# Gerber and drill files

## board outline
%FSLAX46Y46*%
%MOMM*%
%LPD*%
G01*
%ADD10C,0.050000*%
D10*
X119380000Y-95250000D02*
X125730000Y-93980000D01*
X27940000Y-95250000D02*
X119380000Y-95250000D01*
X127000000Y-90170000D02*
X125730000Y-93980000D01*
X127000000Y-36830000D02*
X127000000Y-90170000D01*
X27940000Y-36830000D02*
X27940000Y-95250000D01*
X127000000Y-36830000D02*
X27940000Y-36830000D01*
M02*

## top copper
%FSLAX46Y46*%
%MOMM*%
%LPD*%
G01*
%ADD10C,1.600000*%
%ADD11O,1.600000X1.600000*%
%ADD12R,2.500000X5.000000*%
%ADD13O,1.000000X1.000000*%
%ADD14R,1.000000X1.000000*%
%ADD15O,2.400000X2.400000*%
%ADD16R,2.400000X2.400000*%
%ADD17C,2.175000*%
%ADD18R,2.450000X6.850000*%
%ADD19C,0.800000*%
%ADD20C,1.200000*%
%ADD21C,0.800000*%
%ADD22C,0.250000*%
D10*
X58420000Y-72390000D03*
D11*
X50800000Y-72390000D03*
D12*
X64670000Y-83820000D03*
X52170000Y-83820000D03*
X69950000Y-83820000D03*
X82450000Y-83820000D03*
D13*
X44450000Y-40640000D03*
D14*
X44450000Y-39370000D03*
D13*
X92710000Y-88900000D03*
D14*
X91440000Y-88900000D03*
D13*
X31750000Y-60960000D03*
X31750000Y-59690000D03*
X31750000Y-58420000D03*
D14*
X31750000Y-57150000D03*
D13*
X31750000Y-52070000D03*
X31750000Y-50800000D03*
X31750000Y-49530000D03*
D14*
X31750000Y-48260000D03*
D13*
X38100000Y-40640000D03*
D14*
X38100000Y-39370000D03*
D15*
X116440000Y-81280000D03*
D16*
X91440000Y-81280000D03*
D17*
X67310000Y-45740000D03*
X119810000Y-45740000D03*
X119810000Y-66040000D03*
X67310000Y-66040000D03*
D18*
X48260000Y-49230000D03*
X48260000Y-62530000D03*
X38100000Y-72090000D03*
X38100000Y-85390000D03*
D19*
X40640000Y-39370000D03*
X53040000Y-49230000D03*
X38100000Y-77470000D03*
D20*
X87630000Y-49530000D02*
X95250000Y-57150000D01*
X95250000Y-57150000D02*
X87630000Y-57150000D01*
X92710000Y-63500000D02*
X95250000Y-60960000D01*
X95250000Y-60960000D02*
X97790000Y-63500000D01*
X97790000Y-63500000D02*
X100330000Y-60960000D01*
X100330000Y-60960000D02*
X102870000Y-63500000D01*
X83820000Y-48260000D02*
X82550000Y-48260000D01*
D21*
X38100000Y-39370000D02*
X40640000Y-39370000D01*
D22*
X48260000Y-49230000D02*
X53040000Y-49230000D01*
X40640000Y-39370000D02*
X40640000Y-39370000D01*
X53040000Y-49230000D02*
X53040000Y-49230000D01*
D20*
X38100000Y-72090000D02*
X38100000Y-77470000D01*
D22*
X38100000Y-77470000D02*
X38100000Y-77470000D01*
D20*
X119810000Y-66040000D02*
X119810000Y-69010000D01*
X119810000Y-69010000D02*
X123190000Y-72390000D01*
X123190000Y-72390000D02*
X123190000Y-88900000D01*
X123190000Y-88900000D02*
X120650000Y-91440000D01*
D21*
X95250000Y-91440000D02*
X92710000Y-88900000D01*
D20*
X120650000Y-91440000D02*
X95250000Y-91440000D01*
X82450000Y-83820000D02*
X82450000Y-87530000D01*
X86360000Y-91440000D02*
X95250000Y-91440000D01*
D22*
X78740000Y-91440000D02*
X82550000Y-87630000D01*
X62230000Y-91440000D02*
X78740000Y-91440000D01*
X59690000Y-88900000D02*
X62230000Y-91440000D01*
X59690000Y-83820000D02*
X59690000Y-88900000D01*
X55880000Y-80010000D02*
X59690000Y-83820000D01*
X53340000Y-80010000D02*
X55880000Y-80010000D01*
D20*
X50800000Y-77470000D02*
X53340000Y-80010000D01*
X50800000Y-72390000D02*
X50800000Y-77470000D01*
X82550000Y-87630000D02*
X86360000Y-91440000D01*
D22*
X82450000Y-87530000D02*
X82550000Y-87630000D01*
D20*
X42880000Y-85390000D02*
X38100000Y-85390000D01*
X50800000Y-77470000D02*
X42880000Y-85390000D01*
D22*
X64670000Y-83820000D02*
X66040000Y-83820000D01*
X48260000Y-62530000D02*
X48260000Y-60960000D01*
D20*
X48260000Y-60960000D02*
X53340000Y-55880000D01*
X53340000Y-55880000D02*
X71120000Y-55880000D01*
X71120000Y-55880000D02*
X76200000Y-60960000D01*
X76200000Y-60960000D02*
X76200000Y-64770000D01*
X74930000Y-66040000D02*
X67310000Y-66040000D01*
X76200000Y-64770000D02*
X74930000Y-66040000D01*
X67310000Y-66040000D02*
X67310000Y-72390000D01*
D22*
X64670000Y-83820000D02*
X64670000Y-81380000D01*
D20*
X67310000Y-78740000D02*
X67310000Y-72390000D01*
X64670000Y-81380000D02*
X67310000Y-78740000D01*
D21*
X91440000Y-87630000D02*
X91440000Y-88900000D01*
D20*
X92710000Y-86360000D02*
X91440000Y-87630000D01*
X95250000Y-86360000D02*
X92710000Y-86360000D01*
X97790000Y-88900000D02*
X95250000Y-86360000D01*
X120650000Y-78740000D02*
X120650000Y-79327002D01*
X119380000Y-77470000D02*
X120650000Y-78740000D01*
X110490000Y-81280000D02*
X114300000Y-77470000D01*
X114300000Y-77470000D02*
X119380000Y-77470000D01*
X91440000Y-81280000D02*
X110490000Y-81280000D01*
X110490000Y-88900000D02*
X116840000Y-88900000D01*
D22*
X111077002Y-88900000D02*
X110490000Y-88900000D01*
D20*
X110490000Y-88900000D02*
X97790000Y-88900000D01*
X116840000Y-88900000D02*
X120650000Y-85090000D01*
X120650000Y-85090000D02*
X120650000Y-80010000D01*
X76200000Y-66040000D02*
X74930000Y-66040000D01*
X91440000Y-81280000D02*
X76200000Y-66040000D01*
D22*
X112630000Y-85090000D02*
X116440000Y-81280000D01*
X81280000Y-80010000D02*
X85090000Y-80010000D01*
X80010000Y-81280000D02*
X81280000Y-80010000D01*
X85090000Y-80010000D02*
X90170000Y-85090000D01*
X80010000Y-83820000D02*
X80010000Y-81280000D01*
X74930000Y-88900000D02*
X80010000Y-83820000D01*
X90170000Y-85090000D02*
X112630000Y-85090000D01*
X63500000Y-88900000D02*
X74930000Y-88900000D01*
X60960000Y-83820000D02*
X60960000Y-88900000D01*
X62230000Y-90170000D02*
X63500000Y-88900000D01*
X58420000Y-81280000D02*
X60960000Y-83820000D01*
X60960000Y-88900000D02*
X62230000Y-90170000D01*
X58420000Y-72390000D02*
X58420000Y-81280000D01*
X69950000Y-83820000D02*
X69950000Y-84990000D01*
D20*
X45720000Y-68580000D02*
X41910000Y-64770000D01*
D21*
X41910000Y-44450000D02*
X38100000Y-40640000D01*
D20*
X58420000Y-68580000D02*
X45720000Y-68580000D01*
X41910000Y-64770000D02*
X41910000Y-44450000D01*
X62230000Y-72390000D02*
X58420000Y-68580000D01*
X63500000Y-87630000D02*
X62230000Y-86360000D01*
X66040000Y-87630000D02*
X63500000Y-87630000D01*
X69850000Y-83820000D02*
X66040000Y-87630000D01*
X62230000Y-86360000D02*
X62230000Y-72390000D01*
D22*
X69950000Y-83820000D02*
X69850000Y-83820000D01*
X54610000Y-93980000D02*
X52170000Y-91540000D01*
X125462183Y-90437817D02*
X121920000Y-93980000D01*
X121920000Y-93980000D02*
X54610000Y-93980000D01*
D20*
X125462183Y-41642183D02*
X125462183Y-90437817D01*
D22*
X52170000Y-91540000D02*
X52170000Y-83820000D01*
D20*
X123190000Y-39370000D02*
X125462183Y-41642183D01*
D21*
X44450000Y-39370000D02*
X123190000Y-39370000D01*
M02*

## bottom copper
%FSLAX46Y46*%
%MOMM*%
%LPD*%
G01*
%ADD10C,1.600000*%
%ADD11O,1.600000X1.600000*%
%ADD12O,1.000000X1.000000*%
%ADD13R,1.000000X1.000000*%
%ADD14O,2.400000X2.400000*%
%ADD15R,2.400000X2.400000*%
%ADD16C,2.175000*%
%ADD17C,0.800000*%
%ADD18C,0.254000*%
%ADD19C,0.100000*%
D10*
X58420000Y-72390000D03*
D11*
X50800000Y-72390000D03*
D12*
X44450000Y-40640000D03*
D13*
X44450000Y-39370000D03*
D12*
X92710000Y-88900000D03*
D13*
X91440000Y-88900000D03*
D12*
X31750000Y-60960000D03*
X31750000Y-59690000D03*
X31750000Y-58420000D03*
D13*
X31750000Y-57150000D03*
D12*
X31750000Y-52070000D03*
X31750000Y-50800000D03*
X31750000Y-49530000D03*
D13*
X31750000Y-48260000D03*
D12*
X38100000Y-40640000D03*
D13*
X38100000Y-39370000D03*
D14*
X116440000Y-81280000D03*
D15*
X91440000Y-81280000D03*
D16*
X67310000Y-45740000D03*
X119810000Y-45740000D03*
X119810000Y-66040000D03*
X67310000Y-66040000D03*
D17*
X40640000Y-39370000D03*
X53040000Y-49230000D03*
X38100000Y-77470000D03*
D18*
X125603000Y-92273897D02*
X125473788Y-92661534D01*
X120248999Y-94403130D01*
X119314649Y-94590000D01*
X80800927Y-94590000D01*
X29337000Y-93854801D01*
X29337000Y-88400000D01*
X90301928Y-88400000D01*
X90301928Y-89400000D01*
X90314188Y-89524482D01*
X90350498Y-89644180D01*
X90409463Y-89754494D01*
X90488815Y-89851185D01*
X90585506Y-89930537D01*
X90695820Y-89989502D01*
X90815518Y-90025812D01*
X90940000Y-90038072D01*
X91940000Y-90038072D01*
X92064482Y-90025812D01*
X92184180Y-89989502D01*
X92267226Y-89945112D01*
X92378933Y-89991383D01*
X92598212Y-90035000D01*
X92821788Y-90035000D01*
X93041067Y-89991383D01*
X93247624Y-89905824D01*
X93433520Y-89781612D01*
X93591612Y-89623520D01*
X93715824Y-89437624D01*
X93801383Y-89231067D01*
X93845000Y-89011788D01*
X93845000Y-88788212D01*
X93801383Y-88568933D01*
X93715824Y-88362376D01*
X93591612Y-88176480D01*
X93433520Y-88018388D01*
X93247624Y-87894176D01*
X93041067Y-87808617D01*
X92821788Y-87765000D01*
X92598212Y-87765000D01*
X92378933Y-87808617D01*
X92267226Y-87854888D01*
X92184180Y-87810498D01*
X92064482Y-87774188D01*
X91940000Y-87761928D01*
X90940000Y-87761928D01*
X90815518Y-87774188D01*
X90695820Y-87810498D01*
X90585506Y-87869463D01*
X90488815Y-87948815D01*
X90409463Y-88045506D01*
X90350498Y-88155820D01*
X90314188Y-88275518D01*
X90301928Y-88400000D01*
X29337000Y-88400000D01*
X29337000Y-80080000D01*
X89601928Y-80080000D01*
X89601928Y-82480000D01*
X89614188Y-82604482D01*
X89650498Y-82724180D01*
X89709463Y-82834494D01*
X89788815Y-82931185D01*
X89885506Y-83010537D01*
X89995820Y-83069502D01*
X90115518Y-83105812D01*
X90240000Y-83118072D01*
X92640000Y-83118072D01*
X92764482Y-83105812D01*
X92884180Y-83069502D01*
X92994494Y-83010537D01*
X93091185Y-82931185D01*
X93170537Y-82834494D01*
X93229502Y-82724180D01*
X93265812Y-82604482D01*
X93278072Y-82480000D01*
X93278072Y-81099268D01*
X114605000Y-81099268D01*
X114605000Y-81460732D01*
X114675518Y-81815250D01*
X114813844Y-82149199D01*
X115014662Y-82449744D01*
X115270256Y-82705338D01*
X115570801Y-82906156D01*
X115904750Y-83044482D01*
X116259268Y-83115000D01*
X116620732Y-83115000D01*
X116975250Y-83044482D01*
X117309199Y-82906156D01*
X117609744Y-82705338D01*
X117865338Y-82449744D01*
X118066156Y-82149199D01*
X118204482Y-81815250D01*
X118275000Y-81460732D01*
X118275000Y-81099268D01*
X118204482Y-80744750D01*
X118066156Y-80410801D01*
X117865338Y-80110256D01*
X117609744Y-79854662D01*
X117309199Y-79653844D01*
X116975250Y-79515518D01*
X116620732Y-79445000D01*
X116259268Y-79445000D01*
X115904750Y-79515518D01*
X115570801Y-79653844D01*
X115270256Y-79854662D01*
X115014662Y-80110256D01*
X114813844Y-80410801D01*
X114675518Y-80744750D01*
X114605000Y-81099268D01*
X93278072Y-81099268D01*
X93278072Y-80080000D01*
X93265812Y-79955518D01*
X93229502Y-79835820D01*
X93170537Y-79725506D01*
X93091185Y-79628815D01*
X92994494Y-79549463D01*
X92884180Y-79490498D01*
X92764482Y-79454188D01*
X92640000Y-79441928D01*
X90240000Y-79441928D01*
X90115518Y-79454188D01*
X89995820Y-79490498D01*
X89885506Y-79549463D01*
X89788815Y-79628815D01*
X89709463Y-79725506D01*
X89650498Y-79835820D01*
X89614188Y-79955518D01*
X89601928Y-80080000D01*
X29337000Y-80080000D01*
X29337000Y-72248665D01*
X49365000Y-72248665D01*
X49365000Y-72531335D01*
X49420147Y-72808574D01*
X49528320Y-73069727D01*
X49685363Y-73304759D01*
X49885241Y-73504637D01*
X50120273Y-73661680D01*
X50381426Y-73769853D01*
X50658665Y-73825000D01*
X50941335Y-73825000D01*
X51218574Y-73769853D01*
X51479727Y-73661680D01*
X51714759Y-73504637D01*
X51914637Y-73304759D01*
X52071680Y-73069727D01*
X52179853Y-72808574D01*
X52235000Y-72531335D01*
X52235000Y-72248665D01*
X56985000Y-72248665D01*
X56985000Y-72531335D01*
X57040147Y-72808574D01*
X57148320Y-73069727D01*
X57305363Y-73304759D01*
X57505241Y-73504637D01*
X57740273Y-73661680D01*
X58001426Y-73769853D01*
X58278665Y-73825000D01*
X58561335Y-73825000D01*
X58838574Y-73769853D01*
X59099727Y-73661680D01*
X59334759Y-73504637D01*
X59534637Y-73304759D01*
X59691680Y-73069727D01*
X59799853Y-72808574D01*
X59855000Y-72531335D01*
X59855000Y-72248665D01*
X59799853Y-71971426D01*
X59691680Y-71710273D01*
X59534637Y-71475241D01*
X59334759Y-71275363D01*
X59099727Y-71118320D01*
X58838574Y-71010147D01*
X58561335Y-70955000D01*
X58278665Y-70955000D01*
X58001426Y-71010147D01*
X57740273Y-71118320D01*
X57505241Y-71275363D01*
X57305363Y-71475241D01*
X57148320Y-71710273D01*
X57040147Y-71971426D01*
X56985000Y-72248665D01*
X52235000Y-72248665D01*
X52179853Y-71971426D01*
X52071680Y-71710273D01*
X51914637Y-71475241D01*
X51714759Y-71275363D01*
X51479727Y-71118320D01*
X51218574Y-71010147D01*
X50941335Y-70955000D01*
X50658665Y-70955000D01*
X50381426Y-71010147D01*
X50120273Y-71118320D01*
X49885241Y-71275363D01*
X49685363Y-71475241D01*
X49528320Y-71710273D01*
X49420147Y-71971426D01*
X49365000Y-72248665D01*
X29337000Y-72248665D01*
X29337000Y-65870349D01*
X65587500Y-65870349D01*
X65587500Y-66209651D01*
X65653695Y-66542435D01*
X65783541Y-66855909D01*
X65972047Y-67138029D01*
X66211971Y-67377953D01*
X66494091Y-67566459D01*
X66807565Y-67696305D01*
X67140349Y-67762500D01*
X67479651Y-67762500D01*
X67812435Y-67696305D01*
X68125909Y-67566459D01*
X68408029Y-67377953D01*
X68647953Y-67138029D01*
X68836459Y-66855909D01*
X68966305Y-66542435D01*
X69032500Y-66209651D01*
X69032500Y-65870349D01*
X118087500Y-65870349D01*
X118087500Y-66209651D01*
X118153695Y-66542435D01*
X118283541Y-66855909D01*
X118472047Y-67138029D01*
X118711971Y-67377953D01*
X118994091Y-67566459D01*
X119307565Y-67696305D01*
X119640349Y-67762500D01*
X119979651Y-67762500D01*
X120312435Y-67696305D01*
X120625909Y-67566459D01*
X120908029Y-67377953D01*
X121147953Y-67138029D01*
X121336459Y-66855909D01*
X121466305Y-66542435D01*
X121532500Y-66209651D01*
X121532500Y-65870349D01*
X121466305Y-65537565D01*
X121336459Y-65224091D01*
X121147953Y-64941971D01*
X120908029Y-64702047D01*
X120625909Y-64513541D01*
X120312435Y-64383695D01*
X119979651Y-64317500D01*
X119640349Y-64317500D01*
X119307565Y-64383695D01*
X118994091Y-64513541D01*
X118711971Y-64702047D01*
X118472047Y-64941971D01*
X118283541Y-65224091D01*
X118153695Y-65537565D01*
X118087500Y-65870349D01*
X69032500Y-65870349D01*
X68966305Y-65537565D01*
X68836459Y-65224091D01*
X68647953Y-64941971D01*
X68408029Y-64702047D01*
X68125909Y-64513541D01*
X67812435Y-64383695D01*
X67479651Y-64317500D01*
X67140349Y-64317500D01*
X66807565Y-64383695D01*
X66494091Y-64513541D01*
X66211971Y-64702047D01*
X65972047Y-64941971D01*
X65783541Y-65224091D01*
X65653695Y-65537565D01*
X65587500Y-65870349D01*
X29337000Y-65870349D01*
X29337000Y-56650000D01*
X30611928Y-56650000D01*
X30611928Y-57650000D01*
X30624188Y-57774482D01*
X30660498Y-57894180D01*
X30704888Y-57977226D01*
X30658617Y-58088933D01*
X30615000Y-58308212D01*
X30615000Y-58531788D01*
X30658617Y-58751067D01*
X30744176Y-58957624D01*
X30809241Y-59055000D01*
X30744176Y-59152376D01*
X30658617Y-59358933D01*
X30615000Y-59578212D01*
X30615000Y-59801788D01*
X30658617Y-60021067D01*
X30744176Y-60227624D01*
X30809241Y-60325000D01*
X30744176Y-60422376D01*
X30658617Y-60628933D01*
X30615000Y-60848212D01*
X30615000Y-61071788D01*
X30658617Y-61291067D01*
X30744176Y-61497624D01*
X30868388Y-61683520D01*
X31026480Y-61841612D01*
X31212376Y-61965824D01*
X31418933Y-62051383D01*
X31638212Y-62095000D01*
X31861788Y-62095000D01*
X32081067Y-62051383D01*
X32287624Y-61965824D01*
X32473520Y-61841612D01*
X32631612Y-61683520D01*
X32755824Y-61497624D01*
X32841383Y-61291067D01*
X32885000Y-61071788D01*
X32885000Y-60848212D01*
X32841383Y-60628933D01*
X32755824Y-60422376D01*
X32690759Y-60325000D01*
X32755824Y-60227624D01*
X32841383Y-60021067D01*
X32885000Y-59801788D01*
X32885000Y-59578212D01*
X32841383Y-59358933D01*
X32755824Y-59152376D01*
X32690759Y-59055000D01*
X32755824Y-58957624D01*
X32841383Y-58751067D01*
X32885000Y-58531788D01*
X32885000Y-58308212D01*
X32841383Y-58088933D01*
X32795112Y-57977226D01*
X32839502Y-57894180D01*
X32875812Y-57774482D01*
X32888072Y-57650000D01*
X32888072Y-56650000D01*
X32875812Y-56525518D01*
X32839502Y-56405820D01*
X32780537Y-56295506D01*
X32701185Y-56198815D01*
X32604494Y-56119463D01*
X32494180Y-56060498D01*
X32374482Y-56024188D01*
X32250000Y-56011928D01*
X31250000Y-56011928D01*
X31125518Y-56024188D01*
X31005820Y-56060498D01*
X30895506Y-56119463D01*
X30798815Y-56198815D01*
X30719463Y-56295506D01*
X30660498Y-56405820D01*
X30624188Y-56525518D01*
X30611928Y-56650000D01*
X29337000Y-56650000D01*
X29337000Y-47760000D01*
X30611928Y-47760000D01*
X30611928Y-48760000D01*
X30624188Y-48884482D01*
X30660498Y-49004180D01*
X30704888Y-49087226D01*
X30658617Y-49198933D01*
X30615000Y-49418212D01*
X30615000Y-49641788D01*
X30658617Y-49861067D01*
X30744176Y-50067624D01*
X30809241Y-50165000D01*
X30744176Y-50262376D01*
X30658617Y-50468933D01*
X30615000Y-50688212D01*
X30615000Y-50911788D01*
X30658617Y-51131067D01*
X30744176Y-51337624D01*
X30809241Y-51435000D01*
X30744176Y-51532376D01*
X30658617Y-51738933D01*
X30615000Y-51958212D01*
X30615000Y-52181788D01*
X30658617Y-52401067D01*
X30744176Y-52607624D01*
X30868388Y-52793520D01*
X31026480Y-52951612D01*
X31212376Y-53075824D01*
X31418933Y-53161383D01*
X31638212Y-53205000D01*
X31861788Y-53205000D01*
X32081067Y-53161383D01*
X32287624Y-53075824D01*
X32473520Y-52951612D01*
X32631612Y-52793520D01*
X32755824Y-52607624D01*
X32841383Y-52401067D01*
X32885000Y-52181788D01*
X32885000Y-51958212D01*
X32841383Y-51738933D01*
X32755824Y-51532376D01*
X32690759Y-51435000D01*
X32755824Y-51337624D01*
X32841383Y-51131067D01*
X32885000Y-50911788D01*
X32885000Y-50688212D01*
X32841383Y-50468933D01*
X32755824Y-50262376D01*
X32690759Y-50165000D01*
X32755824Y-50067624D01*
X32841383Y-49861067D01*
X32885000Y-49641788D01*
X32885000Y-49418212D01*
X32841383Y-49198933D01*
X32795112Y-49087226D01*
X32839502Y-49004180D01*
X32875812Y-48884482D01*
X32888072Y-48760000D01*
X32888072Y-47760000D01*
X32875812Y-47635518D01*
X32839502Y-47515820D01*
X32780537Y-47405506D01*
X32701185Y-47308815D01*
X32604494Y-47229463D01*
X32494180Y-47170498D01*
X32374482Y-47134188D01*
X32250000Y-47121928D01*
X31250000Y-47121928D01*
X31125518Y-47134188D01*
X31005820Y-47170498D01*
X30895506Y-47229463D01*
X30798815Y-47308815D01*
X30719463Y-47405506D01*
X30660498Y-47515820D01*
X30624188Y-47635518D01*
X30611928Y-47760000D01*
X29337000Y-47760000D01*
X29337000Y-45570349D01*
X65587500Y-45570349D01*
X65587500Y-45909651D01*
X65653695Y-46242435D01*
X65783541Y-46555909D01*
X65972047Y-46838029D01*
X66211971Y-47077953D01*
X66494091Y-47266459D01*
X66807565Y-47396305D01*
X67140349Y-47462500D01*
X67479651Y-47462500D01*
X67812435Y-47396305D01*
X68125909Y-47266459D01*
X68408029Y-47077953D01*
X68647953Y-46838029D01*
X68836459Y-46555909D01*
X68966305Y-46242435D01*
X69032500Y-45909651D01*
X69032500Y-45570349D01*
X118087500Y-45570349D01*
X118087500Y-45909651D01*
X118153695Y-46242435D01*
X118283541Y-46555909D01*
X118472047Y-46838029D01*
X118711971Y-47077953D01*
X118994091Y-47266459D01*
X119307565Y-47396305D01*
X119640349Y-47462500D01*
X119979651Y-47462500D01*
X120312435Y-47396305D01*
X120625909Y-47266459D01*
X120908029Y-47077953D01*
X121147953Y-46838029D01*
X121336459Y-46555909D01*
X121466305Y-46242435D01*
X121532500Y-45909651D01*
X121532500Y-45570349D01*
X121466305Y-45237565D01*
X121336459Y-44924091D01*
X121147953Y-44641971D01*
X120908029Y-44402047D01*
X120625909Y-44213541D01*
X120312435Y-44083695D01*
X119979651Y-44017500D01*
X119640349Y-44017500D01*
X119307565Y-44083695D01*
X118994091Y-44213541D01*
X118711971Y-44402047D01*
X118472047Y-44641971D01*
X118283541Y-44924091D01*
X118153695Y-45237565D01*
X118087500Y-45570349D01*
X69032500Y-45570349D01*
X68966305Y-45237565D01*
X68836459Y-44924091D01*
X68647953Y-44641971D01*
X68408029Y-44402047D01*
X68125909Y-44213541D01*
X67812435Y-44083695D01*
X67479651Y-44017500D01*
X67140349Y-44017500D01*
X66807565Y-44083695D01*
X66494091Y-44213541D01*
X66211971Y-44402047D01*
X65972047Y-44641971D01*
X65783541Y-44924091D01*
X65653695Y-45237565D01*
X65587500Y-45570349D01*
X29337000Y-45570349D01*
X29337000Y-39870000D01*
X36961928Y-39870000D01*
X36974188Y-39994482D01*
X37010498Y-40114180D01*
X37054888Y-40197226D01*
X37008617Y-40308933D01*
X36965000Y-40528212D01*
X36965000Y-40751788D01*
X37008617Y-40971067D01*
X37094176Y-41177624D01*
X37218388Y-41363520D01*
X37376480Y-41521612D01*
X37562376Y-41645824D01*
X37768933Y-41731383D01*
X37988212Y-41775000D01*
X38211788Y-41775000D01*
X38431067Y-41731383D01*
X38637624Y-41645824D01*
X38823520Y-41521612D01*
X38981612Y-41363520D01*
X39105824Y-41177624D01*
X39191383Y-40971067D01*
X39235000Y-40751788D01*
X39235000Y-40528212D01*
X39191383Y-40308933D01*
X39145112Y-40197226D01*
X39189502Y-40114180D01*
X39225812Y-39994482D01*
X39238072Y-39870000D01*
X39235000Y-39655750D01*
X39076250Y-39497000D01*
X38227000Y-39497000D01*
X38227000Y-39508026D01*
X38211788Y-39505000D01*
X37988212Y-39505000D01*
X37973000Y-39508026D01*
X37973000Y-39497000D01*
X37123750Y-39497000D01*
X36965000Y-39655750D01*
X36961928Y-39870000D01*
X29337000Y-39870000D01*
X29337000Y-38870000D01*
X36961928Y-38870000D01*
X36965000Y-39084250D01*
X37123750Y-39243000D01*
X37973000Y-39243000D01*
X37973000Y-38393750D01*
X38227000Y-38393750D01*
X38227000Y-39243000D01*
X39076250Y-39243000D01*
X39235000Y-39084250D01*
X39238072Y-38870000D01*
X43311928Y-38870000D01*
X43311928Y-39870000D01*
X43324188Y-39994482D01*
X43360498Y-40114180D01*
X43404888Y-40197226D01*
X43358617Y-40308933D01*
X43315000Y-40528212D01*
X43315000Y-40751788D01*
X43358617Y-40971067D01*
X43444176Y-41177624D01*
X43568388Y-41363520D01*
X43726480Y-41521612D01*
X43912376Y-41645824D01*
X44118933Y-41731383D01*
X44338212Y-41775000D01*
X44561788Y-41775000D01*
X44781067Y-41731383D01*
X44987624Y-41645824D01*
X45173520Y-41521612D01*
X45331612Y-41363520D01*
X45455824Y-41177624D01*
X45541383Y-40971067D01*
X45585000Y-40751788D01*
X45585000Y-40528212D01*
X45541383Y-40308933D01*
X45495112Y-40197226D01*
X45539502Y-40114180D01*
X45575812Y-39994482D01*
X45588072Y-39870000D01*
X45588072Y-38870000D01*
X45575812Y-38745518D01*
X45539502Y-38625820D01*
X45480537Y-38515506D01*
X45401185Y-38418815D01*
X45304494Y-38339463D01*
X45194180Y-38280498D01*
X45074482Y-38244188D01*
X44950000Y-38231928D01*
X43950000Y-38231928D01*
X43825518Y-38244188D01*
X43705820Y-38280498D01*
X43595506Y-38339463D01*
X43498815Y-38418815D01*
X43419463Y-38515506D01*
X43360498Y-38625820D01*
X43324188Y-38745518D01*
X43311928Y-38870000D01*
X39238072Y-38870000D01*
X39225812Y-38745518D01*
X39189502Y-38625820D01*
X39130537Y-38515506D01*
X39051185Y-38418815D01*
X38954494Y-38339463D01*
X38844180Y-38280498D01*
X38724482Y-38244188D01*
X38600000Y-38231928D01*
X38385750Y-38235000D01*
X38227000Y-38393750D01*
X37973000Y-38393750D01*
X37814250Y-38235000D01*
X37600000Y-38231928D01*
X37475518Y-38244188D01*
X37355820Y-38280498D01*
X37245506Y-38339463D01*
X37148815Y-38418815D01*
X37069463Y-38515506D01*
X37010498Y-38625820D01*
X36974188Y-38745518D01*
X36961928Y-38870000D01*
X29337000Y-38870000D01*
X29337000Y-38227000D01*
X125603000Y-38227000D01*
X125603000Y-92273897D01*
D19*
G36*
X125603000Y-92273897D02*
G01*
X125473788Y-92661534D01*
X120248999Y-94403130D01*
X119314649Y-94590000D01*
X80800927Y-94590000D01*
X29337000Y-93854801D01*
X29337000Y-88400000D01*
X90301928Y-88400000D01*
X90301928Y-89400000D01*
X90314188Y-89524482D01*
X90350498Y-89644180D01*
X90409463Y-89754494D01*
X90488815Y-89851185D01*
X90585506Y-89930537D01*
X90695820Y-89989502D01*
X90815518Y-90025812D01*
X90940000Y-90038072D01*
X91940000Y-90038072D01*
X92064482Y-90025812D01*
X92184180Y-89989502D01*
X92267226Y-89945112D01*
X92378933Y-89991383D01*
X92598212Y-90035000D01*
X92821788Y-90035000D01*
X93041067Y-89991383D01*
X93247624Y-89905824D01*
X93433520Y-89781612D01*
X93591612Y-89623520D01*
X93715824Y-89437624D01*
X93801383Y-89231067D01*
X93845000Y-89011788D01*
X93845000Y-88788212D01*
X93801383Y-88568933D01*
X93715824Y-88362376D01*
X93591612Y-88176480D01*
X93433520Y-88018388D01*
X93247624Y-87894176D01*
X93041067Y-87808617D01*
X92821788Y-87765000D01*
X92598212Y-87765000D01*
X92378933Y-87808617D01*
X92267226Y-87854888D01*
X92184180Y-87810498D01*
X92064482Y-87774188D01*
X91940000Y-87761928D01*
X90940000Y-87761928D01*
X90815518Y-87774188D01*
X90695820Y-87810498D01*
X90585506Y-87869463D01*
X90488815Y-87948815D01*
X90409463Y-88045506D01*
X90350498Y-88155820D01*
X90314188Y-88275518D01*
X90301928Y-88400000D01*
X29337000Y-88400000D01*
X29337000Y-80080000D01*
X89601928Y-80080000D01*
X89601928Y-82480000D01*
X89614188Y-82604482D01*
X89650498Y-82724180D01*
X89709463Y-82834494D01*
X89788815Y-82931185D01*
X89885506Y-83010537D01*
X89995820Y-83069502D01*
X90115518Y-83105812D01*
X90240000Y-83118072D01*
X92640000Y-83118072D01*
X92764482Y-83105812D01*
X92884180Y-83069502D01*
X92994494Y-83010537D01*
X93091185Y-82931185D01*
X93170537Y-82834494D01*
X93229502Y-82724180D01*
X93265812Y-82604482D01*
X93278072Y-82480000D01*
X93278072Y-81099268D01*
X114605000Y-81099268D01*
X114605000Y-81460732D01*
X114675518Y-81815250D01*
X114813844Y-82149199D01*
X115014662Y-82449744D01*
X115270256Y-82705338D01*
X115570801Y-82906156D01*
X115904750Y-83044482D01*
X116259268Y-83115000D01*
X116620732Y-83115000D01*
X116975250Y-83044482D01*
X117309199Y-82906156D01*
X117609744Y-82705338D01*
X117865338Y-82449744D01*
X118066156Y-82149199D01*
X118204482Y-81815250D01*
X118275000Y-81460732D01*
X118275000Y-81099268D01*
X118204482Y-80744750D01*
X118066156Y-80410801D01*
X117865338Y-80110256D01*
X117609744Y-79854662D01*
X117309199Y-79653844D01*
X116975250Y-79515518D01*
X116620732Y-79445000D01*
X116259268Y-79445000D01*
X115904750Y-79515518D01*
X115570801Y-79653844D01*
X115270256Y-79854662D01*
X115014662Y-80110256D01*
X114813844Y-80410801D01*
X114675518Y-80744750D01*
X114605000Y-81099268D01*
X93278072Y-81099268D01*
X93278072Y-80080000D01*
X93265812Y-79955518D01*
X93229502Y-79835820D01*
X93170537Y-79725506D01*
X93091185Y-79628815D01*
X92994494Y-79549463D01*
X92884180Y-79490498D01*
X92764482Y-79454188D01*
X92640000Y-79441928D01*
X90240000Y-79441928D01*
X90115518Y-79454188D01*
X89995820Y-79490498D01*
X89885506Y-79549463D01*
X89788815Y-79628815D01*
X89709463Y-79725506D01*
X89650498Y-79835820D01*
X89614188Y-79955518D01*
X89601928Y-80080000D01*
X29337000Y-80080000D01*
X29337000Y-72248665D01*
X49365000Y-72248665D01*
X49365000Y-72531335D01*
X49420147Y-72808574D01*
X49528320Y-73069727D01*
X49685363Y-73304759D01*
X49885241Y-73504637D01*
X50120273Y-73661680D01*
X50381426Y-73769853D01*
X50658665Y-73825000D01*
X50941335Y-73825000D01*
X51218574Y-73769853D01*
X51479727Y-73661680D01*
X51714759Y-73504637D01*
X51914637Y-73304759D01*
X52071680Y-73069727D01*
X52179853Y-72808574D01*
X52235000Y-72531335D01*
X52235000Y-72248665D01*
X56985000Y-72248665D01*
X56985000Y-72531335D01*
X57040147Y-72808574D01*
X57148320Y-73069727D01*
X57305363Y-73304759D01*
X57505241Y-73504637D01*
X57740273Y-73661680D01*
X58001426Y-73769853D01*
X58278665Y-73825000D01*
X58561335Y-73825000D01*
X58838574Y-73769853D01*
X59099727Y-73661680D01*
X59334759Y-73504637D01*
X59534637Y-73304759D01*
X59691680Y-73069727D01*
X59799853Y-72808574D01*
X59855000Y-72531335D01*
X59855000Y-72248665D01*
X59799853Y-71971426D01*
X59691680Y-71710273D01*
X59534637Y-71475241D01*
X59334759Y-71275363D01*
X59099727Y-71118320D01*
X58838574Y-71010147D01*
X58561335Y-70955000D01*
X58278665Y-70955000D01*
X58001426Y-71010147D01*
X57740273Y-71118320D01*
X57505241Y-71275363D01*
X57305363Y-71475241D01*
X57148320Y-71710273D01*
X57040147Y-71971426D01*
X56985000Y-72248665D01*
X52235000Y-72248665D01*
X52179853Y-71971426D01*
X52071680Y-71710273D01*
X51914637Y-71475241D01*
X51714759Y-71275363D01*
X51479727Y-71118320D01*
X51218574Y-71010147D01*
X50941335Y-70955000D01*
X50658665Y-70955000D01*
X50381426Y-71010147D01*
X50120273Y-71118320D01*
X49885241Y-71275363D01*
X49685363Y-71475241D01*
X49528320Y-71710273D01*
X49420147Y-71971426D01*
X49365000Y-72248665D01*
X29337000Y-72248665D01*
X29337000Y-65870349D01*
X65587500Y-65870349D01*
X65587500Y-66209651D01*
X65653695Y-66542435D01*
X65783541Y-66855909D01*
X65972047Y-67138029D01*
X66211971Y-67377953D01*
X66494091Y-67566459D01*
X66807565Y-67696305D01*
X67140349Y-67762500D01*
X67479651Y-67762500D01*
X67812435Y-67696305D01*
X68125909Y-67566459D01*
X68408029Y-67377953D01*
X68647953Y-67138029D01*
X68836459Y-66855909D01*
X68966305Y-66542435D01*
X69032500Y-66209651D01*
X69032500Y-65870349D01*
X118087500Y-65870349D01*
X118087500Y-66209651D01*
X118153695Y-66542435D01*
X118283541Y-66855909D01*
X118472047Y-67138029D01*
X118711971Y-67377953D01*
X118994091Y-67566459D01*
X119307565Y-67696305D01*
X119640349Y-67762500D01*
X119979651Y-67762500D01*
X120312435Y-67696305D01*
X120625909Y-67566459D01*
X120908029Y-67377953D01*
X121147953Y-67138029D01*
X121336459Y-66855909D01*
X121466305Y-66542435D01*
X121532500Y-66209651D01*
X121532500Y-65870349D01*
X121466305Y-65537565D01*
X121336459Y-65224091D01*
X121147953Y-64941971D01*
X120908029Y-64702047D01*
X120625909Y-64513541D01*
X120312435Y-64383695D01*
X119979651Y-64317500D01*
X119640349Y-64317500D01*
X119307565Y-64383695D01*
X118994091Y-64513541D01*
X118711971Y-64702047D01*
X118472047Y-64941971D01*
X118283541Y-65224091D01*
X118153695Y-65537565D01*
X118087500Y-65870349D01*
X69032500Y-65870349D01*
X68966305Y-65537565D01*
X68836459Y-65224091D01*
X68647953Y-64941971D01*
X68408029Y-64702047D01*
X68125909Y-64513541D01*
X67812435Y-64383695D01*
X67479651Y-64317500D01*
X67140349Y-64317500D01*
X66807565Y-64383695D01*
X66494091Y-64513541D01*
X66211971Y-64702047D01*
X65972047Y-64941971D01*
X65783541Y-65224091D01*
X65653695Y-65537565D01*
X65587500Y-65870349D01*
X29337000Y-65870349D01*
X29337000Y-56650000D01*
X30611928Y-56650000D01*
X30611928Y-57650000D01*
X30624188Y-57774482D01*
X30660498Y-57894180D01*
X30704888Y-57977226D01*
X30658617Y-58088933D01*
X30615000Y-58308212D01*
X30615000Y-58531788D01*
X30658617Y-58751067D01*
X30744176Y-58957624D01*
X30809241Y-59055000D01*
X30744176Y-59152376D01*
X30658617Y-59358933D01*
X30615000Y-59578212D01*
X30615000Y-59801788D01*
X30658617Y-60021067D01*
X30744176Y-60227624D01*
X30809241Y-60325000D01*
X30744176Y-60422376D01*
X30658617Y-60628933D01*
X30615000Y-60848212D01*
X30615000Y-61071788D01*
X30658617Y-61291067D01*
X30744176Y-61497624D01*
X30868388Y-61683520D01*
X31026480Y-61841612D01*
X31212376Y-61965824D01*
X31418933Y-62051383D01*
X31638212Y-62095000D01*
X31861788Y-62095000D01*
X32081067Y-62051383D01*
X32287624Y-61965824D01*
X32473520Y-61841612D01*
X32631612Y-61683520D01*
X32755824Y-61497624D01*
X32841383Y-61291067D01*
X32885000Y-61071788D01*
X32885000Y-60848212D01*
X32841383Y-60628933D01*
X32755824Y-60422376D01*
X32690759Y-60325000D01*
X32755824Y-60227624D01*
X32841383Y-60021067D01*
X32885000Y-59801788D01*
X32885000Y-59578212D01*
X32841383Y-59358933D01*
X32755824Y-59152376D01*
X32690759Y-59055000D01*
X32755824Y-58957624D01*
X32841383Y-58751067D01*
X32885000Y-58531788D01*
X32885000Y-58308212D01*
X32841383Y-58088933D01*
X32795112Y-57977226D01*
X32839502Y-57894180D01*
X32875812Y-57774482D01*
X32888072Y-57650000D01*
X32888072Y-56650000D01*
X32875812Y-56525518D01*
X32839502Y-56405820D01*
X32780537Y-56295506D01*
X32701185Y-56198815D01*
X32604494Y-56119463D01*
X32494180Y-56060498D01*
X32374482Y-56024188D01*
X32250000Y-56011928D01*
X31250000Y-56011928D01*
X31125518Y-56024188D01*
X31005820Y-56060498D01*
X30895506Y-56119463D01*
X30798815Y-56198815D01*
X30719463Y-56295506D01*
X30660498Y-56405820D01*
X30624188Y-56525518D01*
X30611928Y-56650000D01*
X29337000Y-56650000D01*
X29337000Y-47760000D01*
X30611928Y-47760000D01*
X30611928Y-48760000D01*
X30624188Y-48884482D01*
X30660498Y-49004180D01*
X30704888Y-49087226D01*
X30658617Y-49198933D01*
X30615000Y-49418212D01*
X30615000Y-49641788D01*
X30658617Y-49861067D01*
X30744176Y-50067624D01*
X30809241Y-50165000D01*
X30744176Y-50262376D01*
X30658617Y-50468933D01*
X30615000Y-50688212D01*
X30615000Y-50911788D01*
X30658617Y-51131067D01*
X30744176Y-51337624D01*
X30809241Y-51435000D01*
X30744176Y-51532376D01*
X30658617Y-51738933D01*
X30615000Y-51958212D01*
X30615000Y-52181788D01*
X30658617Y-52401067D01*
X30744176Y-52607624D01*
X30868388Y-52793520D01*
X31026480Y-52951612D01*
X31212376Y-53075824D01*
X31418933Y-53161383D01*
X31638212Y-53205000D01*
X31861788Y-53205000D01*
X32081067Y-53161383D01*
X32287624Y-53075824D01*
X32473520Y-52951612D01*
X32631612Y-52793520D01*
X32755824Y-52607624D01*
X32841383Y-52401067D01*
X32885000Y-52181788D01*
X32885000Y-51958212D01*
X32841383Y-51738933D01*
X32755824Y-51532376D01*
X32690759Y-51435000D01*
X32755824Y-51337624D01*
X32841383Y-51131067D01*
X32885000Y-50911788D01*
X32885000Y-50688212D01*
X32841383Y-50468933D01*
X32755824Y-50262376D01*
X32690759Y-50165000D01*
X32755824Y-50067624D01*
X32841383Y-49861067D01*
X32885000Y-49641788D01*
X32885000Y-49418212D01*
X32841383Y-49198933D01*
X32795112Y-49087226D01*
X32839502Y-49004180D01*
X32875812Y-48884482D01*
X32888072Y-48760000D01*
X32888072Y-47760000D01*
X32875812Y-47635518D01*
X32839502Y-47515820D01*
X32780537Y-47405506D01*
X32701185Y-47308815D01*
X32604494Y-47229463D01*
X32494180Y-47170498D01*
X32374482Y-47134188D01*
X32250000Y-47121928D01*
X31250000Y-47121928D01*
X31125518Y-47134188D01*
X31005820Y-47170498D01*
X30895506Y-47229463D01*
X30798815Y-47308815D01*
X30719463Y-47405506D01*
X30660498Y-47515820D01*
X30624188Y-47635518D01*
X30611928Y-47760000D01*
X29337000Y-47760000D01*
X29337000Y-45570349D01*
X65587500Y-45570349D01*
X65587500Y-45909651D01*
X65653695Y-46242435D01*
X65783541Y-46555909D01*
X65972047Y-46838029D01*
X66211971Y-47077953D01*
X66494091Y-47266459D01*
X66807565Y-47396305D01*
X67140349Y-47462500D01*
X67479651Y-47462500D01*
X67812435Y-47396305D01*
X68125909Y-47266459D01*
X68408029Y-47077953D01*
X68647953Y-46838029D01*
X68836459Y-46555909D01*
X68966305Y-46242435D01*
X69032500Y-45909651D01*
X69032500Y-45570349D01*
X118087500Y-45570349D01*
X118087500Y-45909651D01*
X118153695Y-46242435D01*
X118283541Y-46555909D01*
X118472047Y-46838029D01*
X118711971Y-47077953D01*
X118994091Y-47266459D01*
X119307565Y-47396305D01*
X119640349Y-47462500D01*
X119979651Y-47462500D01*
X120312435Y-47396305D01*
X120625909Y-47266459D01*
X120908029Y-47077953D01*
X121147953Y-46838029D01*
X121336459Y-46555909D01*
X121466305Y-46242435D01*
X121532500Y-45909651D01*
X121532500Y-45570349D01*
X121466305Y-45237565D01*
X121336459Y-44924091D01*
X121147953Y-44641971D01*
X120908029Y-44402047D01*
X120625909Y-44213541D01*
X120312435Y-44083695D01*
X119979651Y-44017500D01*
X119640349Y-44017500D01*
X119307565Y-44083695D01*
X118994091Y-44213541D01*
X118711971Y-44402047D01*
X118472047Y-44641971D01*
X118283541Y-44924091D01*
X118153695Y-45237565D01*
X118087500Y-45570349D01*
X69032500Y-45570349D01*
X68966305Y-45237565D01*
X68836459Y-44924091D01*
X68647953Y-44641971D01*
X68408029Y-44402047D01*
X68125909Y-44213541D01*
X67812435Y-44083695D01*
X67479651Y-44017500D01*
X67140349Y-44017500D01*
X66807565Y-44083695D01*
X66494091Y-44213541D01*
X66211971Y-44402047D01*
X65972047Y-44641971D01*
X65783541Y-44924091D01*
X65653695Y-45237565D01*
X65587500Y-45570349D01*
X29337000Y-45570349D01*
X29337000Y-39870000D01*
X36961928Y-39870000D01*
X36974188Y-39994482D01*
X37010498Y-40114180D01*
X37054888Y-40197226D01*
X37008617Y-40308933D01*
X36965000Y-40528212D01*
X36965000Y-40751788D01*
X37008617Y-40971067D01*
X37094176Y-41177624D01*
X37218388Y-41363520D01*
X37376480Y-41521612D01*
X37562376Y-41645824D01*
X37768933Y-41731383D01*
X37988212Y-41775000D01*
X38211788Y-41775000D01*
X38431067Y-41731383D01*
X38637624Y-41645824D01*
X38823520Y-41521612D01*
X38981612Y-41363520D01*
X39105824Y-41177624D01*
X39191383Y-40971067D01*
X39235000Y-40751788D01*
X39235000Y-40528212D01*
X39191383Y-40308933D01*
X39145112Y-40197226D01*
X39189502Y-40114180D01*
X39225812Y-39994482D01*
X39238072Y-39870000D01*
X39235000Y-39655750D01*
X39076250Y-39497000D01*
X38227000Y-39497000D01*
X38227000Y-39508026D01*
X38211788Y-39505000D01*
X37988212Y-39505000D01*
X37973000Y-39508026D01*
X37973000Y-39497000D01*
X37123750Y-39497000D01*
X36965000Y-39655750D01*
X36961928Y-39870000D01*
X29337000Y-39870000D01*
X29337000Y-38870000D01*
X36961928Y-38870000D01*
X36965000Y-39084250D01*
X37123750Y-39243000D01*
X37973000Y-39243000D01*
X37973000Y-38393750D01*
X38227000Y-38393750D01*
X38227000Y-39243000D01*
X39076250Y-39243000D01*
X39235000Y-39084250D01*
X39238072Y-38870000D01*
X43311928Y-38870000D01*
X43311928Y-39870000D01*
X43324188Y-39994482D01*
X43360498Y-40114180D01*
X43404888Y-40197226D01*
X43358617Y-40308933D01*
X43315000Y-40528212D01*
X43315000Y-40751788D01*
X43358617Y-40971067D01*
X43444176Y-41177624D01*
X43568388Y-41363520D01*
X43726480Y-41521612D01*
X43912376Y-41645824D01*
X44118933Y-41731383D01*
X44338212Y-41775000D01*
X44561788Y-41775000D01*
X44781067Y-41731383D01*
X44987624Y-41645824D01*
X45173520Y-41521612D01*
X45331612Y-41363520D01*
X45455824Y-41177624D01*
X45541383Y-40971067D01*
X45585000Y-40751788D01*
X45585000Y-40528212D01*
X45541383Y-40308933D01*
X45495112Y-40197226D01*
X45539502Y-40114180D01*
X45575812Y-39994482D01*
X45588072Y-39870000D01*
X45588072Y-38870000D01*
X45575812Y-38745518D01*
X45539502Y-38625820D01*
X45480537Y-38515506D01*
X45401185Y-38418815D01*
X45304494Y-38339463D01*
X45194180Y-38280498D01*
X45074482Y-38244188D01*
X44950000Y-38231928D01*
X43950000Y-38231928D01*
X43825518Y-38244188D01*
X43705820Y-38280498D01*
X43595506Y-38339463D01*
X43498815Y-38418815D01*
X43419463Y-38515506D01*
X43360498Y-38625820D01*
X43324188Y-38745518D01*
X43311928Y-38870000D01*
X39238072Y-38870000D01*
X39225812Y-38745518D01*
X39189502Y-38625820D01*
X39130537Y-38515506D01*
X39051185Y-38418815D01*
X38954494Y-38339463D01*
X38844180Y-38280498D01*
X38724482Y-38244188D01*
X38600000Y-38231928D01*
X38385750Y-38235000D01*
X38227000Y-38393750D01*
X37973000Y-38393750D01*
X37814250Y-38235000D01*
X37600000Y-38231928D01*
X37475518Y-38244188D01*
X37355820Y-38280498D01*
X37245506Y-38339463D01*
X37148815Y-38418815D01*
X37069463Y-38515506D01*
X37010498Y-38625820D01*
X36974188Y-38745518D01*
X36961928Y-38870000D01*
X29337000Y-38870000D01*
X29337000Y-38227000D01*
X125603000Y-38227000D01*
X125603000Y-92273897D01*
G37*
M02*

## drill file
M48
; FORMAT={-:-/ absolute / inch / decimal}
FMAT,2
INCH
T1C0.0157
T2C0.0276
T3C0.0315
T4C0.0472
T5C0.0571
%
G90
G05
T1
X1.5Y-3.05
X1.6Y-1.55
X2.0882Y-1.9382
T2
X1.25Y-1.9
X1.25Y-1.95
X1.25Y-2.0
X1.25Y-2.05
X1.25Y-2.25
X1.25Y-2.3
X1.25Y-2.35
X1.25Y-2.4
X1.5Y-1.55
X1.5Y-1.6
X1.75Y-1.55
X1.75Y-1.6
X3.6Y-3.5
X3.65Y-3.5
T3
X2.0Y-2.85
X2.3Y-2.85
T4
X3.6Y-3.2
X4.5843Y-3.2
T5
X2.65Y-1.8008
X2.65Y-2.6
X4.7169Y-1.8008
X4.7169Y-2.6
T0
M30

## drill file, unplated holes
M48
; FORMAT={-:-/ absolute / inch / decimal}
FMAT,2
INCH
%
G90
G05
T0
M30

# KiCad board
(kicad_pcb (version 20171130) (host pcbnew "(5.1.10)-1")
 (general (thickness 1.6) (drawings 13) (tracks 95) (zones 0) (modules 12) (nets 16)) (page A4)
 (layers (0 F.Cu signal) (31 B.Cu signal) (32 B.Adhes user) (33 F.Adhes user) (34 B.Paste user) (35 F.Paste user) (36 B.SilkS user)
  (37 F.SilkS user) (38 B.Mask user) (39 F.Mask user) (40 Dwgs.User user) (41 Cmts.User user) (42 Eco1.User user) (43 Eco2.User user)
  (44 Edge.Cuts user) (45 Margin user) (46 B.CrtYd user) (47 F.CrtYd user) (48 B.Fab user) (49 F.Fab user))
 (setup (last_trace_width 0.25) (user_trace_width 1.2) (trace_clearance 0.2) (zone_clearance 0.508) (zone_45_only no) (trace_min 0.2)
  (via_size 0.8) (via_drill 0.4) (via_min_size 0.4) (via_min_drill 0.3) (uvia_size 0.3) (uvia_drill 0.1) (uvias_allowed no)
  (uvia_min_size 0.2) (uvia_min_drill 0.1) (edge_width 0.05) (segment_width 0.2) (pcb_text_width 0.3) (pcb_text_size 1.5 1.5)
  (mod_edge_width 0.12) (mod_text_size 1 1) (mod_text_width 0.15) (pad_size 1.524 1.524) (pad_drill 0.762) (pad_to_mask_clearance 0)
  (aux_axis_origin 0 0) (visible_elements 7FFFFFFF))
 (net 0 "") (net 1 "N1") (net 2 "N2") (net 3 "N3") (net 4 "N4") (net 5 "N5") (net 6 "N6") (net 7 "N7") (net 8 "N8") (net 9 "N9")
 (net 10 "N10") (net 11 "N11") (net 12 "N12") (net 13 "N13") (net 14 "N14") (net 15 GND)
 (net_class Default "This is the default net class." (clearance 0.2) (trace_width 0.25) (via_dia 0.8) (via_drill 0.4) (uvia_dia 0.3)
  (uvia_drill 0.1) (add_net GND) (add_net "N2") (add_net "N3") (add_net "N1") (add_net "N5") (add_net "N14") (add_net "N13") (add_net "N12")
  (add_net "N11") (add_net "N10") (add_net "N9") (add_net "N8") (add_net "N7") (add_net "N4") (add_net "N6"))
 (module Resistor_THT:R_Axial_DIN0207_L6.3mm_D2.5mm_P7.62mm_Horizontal (layer F.Cu) (at 58.42 72.39 180)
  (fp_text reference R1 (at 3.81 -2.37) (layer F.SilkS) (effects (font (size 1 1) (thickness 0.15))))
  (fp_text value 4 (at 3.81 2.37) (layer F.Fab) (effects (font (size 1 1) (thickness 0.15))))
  (pad 1 thru_hole circle (at 0 0 180) (size 1.6 1.6) (drill 0.8) (layers *.Cu *.Mask) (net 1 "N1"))
  (pad 2 thru_hole oval (at 7.62 0 180) (size 1.6 1.6) (drill 0.8) (layers *.Cu *.Mask) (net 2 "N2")))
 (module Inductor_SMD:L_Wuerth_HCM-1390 (layer F.Cu) (at 58.42 83.82)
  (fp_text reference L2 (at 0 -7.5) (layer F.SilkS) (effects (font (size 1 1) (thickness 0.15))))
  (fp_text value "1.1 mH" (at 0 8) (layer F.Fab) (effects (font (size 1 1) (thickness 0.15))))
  (pad 2 smd rect (at 6.25 0) (size 2.5 5) (layers F.Cu F.Paste F.Mask) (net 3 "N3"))
  (pad 1 smd rect (at -6.25 0) (size 2.5 5) (layers F.Cu F.Paste F.Mask) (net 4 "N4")))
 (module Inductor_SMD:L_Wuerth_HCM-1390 (layer F.Cu) (at 76.2 83.82 180)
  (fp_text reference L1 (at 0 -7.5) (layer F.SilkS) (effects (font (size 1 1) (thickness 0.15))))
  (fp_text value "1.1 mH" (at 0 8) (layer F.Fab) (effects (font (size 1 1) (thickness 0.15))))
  (pad 2 smd rect (at 6.25 0 180) (size 2.5 5) (layers F.Cu F.Paste F.Mask) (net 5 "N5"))
  (pad 1 smd rect (at -6.25 0 180) (size 2.5 5) (layers F.Cu F.Paste F.Mask) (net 2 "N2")))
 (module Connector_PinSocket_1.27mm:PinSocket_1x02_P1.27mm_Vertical (layer F.Cu) (at 44.45 39.37)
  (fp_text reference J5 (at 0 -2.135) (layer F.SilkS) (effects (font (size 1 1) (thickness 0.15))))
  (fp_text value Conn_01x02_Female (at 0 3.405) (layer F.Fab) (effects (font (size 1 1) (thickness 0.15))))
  (pad 2 thru_hole oval (at 0 1.27) (size 1 1) (drill 0.7) (layers *.Cu *.Mask) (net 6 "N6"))
  (pad 1 thru_hole rect (at 0 0) (size 1 1) (drill 0.7) (layers *.Cu *.Mask) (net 4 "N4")))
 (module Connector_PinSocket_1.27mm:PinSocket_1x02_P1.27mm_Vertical (layer F.Cu) (at 91.44 88.9 90)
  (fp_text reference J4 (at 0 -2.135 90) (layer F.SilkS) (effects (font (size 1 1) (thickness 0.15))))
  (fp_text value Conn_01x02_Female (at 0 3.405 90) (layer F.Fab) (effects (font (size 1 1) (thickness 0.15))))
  (pad 2 thru_hole oval (at 0 1.27 90) (size 1 1) (drill 0.7) (layers *.Cu *.Mask) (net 2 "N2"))
  (pad 1 thru_hole rect (at 0 0 90) (size 1 1) (drill 0.7) (layers *.Cu *.Mask) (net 3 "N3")))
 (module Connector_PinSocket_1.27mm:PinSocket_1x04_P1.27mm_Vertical (layer F.Cu) (at 31.75 57.15)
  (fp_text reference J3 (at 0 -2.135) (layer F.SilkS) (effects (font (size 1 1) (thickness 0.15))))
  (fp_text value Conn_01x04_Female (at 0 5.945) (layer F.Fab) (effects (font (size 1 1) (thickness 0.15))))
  (pad 4 thru_hole oval (at 0 3.81) (size 1 1) (drill 0.7) (layers *.Cu *.Mask) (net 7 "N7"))
  (pad 3 thru_hole oval (at 0 2.54) (size 1 1) (drill 0.7) (layers *.Cu *.Mask) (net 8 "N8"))
  (pad 2 thru_hole oval (at 0 1.27) (size 1 1) (drill 0.7) (layers *.Cu *.Mask) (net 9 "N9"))
  (pad 1 thru_hole rect (at 0 0) (size 1 1) (drill 0.7) (layers *.Cu *.Mask) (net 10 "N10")))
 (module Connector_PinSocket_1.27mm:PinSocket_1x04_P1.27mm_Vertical (layer F.Cu) (at 31.75 48.26)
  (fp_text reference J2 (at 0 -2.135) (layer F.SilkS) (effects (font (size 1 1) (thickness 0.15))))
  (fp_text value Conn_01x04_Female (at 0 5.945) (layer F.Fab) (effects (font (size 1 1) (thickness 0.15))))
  (pad 4 thru_hole oval (at 0 3.81) (size 1 1) (drill 0.7) (layers *.Cu *.Mask) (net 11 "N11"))
  (pad 3 thru_hole oval (at 0 2.54) (size 1 1) (drill 0.7) (layers *.Cu *.Mask) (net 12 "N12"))
  (pad 2 thru_hole oval (at 0 1.27) (size 1 1) (drill 0.7) (layers *.Cu *.Mask) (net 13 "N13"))
  (pad 1 thru_hole rect (at 0 0) (size 1 1) (drill 0.7) (layers *.Cu *.Mask) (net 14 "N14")))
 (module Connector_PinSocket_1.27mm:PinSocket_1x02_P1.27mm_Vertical (layer F.Cu) (at 38.1 39.37)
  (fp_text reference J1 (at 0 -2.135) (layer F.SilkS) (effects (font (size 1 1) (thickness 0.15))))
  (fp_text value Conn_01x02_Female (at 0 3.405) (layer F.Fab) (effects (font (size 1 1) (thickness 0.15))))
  (pad 2 thru_hole oval (at 0 1.27) (size 1 1) (drill 0.7) (layers *.Cu *.Mask) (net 5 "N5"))
  (pad 1 thru_hole rect (at 0 0) (size 1 1) (drill 0.7) (layers *.Cu *.Mask) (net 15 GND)))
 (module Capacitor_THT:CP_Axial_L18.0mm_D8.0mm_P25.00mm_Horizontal (layer F.Cu) (at 91.44 81.28)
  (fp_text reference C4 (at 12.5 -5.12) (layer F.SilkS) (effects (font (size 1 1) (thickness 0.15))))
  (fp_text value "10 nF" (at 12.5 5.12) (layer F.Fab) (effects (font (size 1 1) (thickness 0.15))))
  (pad 2 thru_hole oval (at 25 0) (size 2.4 2.4) (drill 1.2) (layers *.Cu *.Mask) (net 1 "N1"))
  (pad 1 thru_hole rect (at 0 0) (size 2.4 2.4) (drill 1.2) (layers *.Cu *.Mask) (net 3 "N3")))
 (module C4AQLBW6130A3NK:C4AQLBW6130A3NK (layer F.Cu) (at 67.31 66.04)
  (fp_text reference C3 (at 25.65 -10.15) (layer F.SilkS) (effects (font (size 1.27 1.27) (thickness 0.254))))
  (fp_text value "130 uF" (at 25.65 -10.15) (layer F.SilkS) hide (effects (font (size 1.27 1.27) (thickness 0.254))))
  (pad 4 thru_hole circle (at 0 -20.3 90) (size 2.175 2.175) (drill 1.45) (layers *.Cu *.Mask F.SilkS))
  (pad 3 thru_hole circle (at 52.5 -20.3 90) (size 2.175 2.175) (drill 1.45) (layers *.Cu *.Mask F.SilkS))
  (pad 2 thru_hole circle (at 52.5 0 90) (size 2.175 2.175) (drill 1.45) (layers *.Cu *.Mask F.SilkS) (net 2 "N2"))
  (pad 1 thru_hole circle (at 0 0 90) (size 2.175 2.175) (drill 1.45) (layers *.Cu *.Mask F.SilkS) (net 3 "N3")))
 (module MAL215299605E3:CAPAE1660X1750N (layer F.Cu) (at 48.26 55.88 90)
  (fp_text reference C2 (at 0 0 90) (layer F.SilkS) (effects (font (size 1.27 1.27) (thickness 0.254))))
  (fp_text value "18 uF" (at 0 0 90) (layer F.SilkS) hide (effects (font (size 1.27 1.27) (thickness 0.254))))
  (pad 2 smd rect (at 6.65 0 180) (size 2.45 6.85) (layers F.Cu F.Paste F.Mask) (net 15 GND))
  (pad 1 smd rect (at -6.65 0 180) (size 2.45 6.85) (layers F.Cu F.Paste F.Mask) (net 3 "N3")))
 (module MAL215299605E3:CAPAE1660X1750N (layer F.Cu) (at 38.1 78.74 90)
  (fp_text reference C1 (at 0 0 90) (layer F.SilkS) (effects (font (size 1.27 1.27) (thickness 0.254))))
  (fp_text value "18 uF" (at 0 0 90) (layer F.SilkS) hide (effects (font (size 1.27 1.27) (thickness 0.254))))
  (pad 2 smd rect (at 6.65 0 180) (size 2.45 6.85) (layers F.Cu F.Paste F.Mask) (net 15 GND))
  (pad 1 smd rect (at -6.65 0 180) (size 2.45 6.85) (layers F.Cu F.Paste F.Mask) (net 2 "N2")))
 (gr_line (start 119.38 95.25) (end 125.73 93.98) (layer Edge.Cuts) (width 0.05))
 (gr_line (start 27.94 95.25) (end 119.38 95.25) (layer Edge.Cuts) (width 0.05))
 (gr_line (start 127 90.17) (end 125.73 93.98) (layer Edge.Cuts) (width 0.05))
 (gr_line (start 127 36.83) (end 127 90.17) (layer Edge.Cuts) (width 0.05))
 (gr_line (start 27.94 36.83) (end 27.94 95.25) (layer Edge.Cuts) (width 0.05))
 (gr_line (start 127 36.83) (end 27.94 36.83) (layer Edge.Cuts) (width 0.05))
 (segment (start 87.63 49.53) (end 95.25 57.15) (width 1.2) (layer F.Cu) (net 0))
 (segment (start 95.25 57.15) (end 87.63 57.15) (width 1.2) (layer F.Cu) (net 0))
 (segment (start 92.71 63.5) (end 95.25 60.96) (width 1.2) (layer F.Cu) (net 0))
 (segment (start 95.25 60.96) (end 97.79 63.5) (width 1.2) (layer F.Cu) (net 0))
 (segment (start 97.79 63.5) (end 100.33 60.96) (width 1.2) (layer F.Cu) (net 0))
 (segment (start 100.33 60.96) (end 102.87 63.5) (width 1.2) (layer F.Cu) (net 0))
 (segment (start 83.82 48.26) (end 82.55 48.26) (width 1.2) (layer F.Cu) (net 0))
 (segment (start 38.1 39.37) (end 40.64 39.37) (width 0.8) (layer F.Cu) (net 15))
 (segment (start 48.26 49.23) (end 53.04 49.23) (width 0.25) (layer F.Cu) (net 15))
 (segment (start 40.64 39.37) (end 40.64 39.37) (width 0.25) (layer F.Cu) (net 15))
 (via (at 40.64 39.37) (size 0.8) (drill 0.4) (layers F.Cu B.Cu) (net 15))
 (segment (start 53.04 49.23) (end 53.04 49.23) (width 0.25) (layer F.Cu) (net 15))
 (via (at 53.04 49.23) (size 0.8) (drill 0.4) (layers F.Cu B.Cu) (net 15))
 (segment (start 38.1 72.09) (end 38.1 77.47) (width 1.2) (layer F.Cu) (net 15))
 (segment (start 38.1 77.47) (end 38.1 77.47) (width 0.25) (layer F.Cu) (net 15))
 (via (at 38.1 77.47) (size 0.8) (drill 0.4) (layers F.Cu B.Cu) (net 15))
 (segment (start 119.81 66.04) (end 119.81 69.01) (width 1.2) (layer F.Cu) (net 2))
 (segment (start 119.81 69.01) (end 123.19 72.39) (width 1.2) (layer F.Cu) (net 2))
 (segment (start 123.19 72.39) (end 123.19 88.9) (width 1.2) (layer F.Cu) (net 2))
 (segment (start 123.19 88.9) (end 120.65 91.44) (width 1.2) (layer F.Cu) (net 2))
 (segment (start 95.25 91.44) (end 92.71 88.9) (width 0.8) (layer F.Cu) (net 2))
 (segment (start 120.65 91.44) (end 95.25 91.44) (width 1.2) (layer F.Cu) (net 2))
 (segment (start 82.45 83.82) (end 82.45 87.53) (width 1.2) (layer F.Cu) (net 2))
 (segment (start 86.36 91.44) (end 95.25 91.44) (width 1.2) (layer F.Cu) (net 2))
 (segment (start 78.74 91.44) (end 82.55 87.63) (width 0.25) (layer F.Cu) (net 2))
 (segment (start 62.23 91.44) (end 78.74 91.44) (width 0.25) (layer F.Cu) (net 2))
 (segment (start 59.69 88.9) (end 62.23 91.44) (width 0.25) (layer F.Cu) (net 2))
 (segment (start 59.69 83.82) (end 59.69 88.9) (width 0.25) (layer F.Cu) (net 2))
 (segment (start 55.88 80.01) (end 59.69 83.82) (width 0.25) (layer F.Cu) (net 2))
 (segment (start 53.34 80.01) (end 55.88 80.01) (width 0.25) (layer F.Cu) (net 2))
 (segment (start 50.8 77.47) (end 53.34 80.01) (width 1.2) (layer F.Cu) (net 2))
 (segment (start 50.8 72.39) (end 50.8 77.47) (width 1.2) (layer F.Cu) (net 2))
 (segment (start 82.55 87.63) (end 86.36 91.44) (width 1.2) (layer F.Cu) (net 2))
 (segment (start 82.45 87.53) (end 82.55 87.63) (width 0.25) (layer F.Cu) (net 2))
 (segment (start 42.88 85.39) (end 38.1 85.39) (width 1.2) (layer F.Cu) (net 2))
 (segment (start 50.8 77.47) (end 42.88 85.39) (width 1.2) (layer F.Cu) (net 2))
 (segment (start 64.67 83.82) (end 66.04 83.82) (width 0.25) (layer F.Cu) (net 3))
 (segment (start 48.26 62.53) (end 48.26 60.96) (width 0.25) (layer F.Cu) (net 3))
 (segment (start 48.26 60.96) (end 53.34 55.88) (width 1.2) (layer F.Cu) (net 3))
 (segment (start 53.34 55.88) (end 71.12 55.88) (width 1.2) (layer F.Cu) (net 3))
 (segment (start 71.12 55.88) (end 76.2 60.96) (width 1.2) (layer F.Cu) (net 3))
 (segment (start 76.2 60.96) (end 76.2 64.77) (width 1.2) (layer F.Cu) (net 3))
 (segment (start 74.93 66.04) (end 67.31 66.04) (width 1.2) (layer F.Cu) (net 3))
 (segment (start 76.2 64.77) (end 74.93 66.04) (width 1.2) (layer F.Cu) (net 3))
 (segment (start 67.31 66.04) (end 67.31 72.39) (width 1.2) (layer F.Cu) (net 3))
 (segment (start 64.67 83.82) (end 64.67 81.38) (width 0.25) (layer F.Cu) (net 3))
 (segment (start 67.31 78.74) (end 67.31 72.39) (width 1.2) (layer F.Cu) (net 3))
 (segment (start 64.67 81.38) (end 67.31 78.74) (width 1.2) (layer F.Cu) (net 3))
 (segment (start 91.44 87.63) (end 91.44 88.9) (width 0.8) (layer F.Cu) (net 3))
 (segment (start 92.71 86.36) (end 91.44 87.63) (width 1.2) (layer F.Cu) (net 3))
 (segment (start 95.25 86.36) (end 92.71 86.36) (width 1.2) (layer F.Cu) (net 3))
 (segment (start 97.79 88.9) (end 95.25 86.36) (width 1.2) (layer F.Cu) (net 3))
 (segment (start 120.65 78.74) (end 120.65 79.327002) (width 1.2) (layer F.Cu) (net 3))
 (segment (start 119.38 77.47) (end 120.65 78.74) (width 1.2) (layer F.Cu) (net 3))
 (segment (start 110.49 81.28) (end 114.3 77.47) (width 1.2) (layer F.Cu) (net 3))
 (segment (start 114.3 77.47) (end 119.38 77.47) (width 1.2) (layer F.Cu) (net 3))
 (segment (start 91.44 81.28) (end 110.49 81.28) (width 1.2) (layer F.Cu) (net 3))
 (segment (start 110.49 88.9) (end 116.84 88.9) (width 1.2) (layer F.Cu) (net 3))
 (segment (start 111.077002 88.9) (end 110.49 88.9) (width 0.25) (layer F.Cu) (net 3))
 (segment (start 110.49 88.9) (end 97.79 88.9) (width 1.2) (layer F.Cu) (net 3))
 (segment (start 116.84 88.9) (end 120.65 85.09) (width 1.2) (layer F.Cu) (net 3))
 (segment (start 120.65 85.09) (end 120.65 80.01) (width 1.2) (layer F.Cu) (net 3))
 (segment (start 76.2 66.04) (end 74.93 66.04) (width 1.2) (layer F.Cu) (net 3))
 (segment (start 91.44 81.28) (end 76.2 66.04) (width 1.2) (layer F.Cu) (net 3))
 (segment (start 112.63 85.09) (end 116.44 81.28) (width 0.25) (layer F.Cu) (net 1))
 (segment (start 81.28 80.01) (end 85.09 80.01) (width 0.25) (layer F.Cu) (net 1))
 (segment (start 80.01 81.28) (end 81.28 80.01) (width 0.25) (layer F.Cu) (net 1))
 (segment (start 85.09 80.01) (end 90.17 85.09) (width 0.25) (layer F.Cu) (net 1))
 (segment (start 80.01 83.82) (end 80.01 81.28) (width 0.25) (layer F.Cu) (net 1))
 (segment (start 74.93 88.9) (end 80.01 83.82) (width 0.25) (layer F.Cu) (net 1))
 (segment (start 90.17 85.09) (end 112.63 85.09) (width 0.25) (layer F.Cu) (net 1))
 (segment (start 63.5 88.9) (end 74.93 88.9) (width 0.25) (layer F.Cu) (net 1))
 (segment (start 60.96 83.82) (end 60.96 88.9) (width 0.25) (layer F.Cu) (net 1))
 (segment (start 62.23 90.17) (end 63.5 88.9) (width 0.25) (layer F.Cu) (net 1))
 (segment (start 58.42 81.28) (end 60.96 83.82) (width 0.25) (layer F.Cu) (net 1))
 (segment (start 60.96 88.9) (end 62.23 90.17) (width 0.25) (layer F.Cu) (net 1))
 (segment (start 58.42 72.39) (end 58.42 81.28) (width 0.25) (layer F.Cu) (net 1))
 (segment (start 69.95 83.82) (end 69.95 84.99) (width 0.25) (layer F.Cu) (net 5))
 (segment (start 45.72 68.58) (end 41.91 64.77) (width 1.2) (layer F.Cu) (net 5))
 (segment (start 41.91 44.45) (end 38.1 40.64) (width 0.8) (layer F.Cu) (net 5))
 (segment (start 58.42 68.58) (end 45.72 68.58) (width 1.2) (layer F.Cu) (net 5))
 (segment (start 41.91 64.77) (end 41.91 44.45) (width 1.2) (layer F.Cu) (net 5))
 (segment (start 62.23 72.39) (end 58.42 68.58) (width 1.2) (layer F.Cu) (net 5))
 (segment (start 63.5 87.63) (end 62.23 86.36) (width 1.2) (layer F.Cu) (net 5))
 (segment (start 66.04 87.63) (end 63.5 87.63) (width 1.2) (layer F.Cu) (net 5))
 (segment (start 69.85 83.82) (end 66.04 87.63) (width 1.2) (layer F.Cu) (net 5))
 (segment (start 62.23 86.36) (end 62.23 72.39) (width 1.2) (layer F.Cu) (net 5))
 (segment (start 69.95 83.82) (end 69.85 83.82) (width 0.25) (layer F.Cu) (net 5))
 (segment (start 54.61 93.98) (end 52.17 91.54) (width 0.25) (layer F.Cu) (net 4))
 (segment (start 125.462183 90.437817) (end 121.92 93.98) (width 0.25) (layer F.Cu) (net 4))
 (segment (start 121.92 93.98) (end 54.61 93.98) (width 0.25) (layer F.Cu) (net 4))
 (segment (start 125.462183 41.642183) (end 125.462183 90.437817) (width 1.2) (layer F.Cu) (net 4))
 (segment (start 52.17 91.54) (end 52.17 83.82) (width 0.25) (layer F.Cu) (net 4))
 (segment (start 123.19 39.37) (end 125.462183 41.642183) (width 1.2) (layer F.Cu) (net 4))
 (segment (start 44.45 39.37) (end 123.19 39.37) (width 0.8) (layer F.Cu) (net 4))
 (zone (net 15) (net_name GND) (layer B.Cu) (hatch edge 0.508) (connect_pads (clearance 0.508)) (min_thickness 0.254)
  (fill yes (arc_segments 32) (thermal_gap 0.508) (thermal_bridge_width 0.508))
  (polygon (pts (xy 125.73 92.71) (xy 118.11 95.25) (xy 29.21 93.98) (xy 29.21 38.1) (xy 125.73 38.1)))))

